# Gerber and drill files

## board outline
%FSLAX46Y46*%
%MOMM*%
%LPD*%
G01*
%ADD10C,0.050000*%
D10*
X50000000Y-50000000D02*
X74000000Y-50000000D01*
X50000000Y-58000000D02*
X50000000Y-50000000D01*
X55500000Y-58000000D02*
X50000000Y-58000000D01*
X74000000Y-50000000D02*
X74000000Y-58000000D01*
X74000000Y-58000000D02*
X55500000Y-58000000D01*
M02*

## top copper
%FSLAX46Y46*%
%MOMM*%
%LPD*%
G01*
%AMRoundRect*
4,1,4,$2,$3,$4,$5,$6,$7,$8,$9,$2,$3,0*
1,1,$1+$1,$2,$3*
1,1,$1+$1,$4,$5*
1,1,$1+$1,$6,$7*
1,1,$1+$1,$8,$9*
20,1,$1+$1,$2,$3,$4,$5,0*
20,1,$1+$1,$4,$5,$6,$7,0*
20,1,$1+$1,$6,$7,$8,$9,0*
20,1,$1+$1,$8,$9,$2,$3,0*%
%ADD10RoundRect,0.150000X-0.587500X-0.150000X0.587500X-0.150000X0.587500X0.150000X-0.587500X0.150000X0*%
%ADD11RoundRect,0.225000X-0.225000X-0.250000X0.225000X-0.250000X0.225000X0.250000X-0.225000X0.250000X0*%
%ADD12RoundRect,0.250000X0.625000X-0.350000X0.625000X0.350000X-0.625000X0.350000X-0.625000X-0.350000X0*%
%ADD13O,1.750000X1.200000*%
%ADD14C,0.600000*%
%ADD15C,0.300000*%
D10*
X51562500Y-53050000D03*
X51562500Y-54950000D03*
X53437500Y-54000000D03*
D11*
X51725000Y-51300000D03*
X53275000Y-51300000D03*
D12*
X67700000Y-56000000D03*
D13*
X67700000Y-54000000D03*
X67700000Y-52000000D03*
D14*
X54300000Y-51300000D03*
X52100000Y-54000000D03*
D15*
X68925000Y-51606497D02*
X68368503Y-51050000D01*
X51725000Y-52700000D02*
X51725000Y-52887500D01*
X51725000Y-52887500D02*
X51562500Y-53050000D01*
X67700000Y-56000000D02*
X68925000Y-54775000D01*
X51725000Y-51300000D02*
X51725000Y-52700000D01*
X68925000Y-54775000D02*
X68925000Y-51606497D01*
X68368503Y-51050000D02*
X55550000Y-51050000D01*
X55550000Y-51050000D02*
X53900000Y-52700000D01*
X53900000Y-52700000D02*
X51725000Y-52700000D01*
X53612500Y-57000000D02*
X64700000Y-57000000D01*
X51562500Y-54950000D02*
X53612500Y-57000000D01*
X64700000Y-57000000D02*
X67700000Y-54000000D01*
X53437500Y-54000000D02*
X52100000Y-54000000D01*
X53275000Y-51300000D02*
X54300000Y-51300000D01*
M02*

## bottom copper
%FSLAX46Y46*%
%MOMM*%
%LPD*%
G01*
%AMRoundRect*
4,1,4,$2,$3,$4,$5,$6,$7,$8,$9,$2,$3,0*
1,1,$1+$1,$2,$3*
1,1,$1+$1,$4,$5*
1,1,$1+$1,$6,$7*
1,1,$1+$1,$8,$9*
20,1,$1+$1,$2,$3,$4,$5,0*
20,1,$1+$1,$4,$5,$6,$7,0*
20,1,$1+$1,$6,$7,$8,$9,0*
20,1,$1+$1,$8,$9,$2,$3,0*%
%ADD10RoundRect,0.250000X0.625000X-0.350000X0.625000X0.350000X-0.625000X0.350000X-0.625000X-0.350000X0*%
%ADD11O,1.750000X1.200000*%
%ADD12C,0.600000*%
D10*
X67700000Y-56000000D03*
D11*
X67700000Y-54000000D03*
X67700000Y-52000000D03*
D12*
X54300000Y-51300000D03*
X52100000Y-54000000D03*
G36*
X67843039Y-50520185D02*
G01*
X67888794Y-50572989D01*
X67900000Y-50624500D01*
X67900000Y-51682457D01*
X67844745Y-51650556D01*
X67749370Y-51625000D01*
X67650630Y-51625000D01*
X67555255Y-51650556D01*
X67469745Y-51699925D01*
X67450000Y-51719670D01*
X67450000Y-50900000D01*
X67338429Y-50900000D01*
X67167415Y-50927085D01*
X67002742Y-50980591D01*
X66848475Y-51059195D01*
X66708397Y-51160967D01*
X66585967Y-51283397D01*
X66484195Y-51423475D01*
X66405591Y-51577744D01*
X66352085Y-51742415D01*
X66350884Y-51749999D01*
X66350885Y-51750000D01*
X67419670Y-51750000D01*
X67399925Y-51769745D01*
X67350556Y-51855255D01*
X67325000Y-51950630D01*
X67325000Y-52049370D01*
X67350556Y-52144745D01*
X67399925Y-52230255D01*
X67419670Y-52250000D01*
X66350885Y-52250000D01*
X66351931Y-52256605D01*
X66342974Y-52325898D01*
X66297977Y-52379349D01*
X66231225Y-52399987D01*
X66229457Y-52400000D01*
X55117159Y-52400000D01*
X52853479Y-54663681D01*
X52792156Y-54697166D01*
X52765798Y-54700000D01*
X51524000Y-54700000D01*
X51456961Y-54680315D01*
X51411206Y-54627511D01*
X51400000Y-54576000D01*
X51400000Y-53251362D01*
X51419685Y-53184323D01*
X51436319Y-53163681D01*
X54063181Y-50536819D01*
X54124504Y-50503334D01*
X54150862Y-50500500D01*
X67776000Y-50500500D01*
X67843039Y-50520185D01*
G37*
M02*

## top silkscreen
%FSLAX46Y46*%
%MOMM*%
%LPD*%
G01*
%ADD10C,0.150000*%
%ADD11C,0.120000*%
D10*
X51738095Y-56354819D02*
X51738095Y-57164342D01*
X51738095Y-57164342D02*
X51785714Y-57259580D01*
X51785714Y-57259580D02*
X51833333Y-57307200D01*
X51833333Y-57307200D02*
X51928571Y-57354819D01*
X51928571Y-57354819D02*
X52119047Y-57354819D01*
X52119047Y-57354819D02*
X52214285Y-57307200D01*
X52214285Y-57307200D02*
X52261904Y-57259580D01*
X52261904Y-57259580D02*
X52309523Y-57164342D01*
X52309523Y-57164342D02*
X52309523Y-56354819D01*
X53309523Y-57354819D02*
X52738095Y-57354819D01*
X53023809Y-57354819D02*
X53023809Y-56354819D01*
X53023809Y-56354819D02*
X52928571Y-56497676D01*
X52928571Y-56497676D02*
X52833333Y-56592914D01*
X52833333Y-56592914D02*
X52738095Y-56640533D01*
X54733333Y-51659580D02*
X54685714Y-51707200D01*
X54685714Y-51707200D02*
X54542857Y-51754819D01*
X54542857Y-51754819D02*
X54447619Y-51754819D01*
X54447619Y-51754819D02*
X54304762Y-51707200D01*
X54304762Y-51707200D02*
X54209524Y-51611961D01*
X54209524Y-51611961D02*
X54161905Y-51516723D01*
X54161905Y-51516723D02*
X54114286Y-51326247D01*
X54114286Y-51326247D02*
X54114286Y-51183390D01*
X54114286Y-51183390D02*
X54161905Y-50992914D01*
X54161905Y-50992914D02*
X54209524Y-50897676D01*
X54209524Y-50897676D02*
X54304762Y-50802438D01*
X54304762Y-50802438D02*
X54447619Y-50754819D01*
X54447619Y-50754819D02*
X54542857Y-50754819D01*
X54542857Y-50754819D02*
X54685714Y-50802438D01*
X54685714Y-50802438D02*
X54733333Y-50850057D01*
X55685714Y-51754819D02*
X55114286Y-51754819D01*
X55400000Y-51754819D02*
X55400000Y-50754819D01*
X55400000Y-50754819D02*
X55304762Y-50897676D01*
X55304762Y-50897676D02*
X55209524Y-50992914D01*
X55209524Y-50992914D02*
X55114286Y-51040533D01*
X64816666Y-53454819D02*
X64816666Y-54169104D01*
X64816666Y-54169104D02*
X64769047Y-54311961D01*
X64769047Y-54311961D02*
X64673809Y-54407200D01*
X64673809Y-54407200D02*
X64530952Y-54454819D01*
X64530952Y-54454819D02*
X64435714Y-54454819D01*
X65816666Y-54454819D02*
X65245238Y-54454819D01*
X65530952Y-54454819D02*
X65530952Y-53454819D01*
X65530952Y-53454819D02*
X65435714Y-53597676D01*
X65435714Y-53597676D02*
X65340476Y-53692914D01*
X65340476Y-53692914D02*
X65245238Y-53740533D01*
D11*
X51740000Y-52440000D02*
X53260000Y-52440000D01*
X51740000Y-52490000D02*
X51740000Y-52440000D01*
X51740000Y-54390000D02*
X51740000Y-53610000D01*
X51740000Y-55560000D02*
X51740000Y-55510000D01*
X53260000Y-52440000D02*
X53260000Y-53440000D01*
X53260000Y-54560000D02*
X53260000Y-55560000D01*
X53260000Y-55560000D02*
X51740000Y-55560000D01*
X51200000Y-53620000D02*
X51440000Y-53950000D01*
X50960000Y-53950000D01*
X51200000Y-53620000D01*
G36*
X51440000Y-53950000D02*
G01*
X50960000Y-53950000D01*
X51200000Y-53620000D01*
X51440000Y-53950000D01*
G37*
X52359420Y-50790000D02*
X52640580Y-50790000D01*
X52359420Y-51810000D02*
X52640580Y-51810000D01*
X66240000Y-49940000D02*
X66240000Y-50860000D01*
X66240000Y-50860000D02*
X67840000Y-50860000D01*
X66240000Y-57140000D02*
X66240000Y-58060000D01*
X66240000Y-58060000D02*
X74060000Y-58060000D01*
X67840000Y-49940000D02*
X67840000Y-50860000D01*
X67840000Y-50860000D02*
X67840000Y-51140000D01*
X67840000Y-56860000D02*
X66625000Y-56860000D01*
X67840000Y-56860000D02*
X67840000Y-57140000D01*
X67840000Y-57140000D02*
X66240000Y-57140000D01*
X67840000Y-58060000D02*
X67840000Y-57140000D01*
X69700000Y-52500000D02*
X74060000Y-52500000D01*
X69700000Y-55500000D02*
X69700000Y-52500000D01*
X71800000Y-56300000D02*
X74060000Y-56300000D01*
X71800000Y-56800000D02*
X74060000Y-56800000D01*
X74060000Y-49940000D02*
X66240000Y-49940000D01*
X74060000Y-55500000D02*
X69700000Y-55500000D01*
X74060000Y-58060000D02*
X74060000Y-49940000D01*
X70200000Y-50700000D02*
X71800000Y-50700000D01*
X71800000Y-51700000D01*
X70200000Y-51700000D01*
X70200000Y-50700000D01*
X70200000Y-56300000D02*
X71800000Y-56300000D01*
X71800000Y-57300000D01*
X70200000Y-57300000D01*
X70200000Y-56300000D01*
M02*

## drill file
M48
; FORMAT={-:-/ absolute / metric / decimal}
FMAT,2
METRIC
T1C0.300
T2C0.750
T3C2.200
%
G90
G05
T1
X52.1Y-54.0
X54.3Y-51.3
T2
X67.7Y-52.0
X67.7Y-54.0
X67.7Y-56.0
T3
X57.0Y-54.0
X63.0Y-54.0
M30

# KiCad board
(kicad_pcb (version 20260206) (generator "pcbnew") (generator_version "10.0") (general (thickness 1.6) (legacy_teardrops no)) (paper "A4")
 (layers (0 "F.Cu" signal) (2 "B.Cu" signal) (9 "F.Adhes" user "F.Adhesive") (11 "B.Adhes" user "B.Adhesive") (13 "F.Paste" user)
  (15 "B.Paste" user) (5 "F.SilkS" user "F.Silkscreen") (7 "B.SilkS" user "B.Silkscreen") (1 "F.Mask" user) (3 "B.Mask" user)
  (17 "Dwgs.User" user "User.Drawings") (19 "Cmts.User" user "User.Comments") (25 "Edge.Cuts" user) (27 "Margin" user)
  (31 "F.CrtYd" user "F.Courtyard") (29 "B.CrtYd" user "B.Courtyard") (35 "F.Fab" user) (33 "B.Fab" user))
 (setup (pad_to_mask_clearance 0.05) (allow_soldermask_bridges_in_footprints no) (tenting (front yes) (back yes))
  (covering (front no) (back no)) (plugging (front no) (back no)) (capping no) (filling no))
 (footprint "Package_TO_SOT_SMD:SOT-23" (layer "F.Cu") (at 52.5 54)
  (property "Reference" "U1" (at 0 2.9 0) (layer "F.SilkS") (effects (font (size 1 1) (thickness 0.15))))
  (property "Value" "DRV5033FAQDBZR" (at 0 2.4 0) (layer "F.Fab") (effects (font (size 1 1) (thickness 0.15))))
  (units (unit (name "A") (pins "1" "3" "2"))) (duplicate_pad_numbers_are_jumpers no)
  (fp_line (start -0.76 -1.56) (end 0.76 -1.56) (stroke (width 0.12) (type solid)) (layer "F.SilkS"))
  (fp_line (start -0.76 -1.51) (end -0.76 -1.56) (stroke (width 0.12) (type solid)) (layer "F.SilkS"))
  (fp_line (start -0.76 0.39) (end -0.76 -0.39) (stroke (width 0.12) (type solid)) (layer "F.SilkS"))
  (fp_line (start -0.76 1.56) (end -0.76 1.51) (stroke (width 0.12) (type solid)) (layer "F.SilkS"))
  (fp_line (start 0.76 -1.56) (end 0.76 -0.56) (stroke (width 0.12) (type solid)) (layer "F.SilkS"))
  (fp_line (start 0.76 0.56) (end 0.76 1.56) (stroke (width 0.12) (type solid)) (layer "F.SilkS"))
  (fp_line (start 0.76 1.56) (end -0.76 1.56) (stroke (width 0.12) (type solid)) (layer "F.SilkS"))
  (fp_poly (pts (xy -1.3 -0.38) (xy -1.06 -0.05) (xy -1.54 -0.05)) (stroke (width 0.12) (type solid)) (fill yes) (layer "F.SilkS"))
  (pad "1" smd roundrect (at -0.9375 -0.95) (size 1.475 0.6) (layers "F.Cu" "F.Mask" "F.Paste") (roundrect_rratio 0.25) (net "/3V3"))
  (pad "2" smd roundrect (at -0.9375 0.95) (size 1.475 0.6) (layers "F.Cu" "F.Mask" "F.Paste") (roundrect_rratio 0.25) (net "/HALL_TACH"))
  (pad "3" smd roundrect (at 0.9375 0) (size 1.475 0.6) (layers "F.Cu" "F.Mask" "F.Paste") (roundrect_rratio 0.25) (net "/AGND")))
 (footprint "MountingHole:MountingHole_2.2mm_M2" (layer "F.Cu") (at 63 54)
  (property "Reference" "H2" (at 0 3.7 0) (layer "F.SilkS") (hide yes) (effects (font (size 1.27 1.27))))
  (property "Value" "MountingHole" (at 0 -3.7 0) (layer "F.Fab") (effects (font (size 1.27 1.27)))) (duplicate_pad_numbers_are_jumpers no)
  (pad "" np_thru_hole circle (at 0 0) (size 2.2 2.2) (drill 2.2) (layers "*.Cu" "*.Mask")))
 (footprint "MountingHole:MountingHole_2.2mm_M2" (layer "F.Cu") (at 57 54)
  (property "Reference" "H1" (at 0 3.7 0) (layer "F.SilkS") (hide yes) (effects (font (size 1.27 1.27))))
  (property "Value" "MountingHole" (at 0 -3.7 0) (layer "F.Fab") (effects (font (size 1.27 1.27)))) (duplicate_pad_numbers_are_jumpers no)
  (pad "" np_thru_hole circle (at 0 0) (size 2.2 2.2) (drill 2.2) (layers "*.Cu" "*.Mask")))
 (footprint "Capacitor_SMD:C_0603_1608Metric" (layer "F.Cu") (at 52.5 51.3)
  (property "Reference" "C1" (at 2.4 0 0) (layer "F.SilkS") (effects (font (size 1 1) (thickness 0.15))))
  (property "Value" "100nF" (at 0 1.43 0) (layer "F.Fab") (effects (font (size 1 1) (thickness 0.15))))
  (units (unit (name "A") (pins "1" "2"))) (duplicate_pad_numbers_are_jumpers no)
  (fp_line (start -0.14058 -0.51) (end 0.14058 -0.51) (stroke (width 0.12) (type solid)) (layer "F.SilkS"))
  (fp_line (start -0.14058 0.51) (end 0.14058 0.51) (stroke (width 0.12) (type solid)) (layer "F.SilkS"))
  (pad "1" smd roundrect (at -0.775 0) (size 0.9 0.95) (layers "F.Cu" "F.Mask" "F.Paste") (roundrect_rratio 0.25) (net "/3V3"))
  (pad "2" smd roundrect (at 0.775 0) (size 0.9 0.95) (layers "F.Cu" "F.Mask" "F.Paste") (roundrect_rratio 0.25) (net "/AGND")))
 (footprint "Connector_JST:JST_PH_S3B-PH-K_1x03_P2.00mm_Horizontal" (layer "F.Cu") (at 67.7 56 90)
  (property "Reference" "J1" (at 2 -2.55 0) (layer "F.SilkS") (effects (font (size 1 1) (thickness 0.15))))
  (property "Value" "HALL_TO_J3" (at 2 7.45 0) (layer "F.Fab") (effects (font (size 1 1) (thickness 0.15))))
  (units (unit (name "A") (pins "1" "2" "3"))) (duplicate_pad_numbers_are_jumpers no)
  (fp_line (start 6.06 -1.46) (end 5.14 -1.46) (stroke (width 0.12) (type solid)) (layer "F.SilkS"))
  (fp_line (start 5.14 -1.46) (end 5.14 0.14) (stroke (width 0.12) (type solid)) (layer "F.SilkS"))
  (fp_line (start -1.14 -1.46) (end -2.06 -1.46) (stroke (width 0.12) (type solid)) (layer "F.SilkS"))
  (fp_line (start -2.06 -1.46) (end -2.06 6.36) (stroke (width 0.12) (type solid)) (layer "F.SilkS"))
  (fp_line (start 6.06 0.14) (end 5.14 0.14) (stroke (width 0.12) (type solid)) (layer "F.SilkS"))
  (fp_line (start 5.14 0.14) (end 4.86 0.14) (stroke (width 0.12) (type solid)) (layer "F.SilkS"))
  (fp_line (start -0.86 0.14) (end -0.86 -1.075) (stroke (width 0.12) (type solid)) (layer "F.SilkS"))
  (fp_line (start -0.86 0.14) (end -1.14 0.14) (stroke (width 0.12) (type solid)) (layer "F.SilkS"))
  (fp_line (start -1.14 0.14) (end -1.14 -1.46) (stroke (width 0.12) (type solid)) (layer "F.SilkS"))
  (fp_line (start -2.06 0.14) (end -1.14 0.14) (stroke (width 0.12) (type solid)) (layer "F.SilkS"))
  (fp_line (start 3.5 2) (end 3.5 6.36) (stroke (width 0.12) (type solid)) (layer "F.SilkS"))
  (fp_line (start 0.5 2) (end 3.5 2) (stroke (width 0.12) (type solid)) (layer "F.SilkS"))
  (fp_line (start -0.3 4.1) (end -0.3 6.36) (stroke (width 0.12) (type solid)) (layer "F.SilkS"))
  (fp_line (start -0.8 4.1) (end -0.8 6.36) (stroke (width 0.12) (type solid)) (layer "F.SilkS"))
  (fp_line (start 6.06 6.36) (end 6.06 -1.46) (stroke (width 0.12) (type solid)) (layer "F.SilkS"))
  (fp_line (start 0.5 6.36) (end 0.5 2) (stroke (width 0.12) (type solid)) (layer "F.SilkS"))
  (fp_line (start -2.06 6.36) (end 6.06 6.36) (stroke (width 0.12) (type solid)) (layer "F.SilkS"))
  (fp_rect (start 4.3 2.5) (end 5.3 4.1) (stroke (width 0.12) (type solid)) (fill no) (layer "F.SilkS"))
  (fp_rect (start -1.3 2.5) (end -0.3 4.1) (stroke (width 0.12) (type solid)) (fill no) (layer "F.SilkS"))
  (pad "1" thru_hole roundrect (at 0 0 90) (size 1.2 1.75) (drill 0.75) (layers "*.Cu" "*.Mask") (remove_unused_layers no)
   (roundrect_rratio 0.208333) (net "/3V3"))
  (pad "2" thru_hole oval (at 2 0 90) (size 1.2 1.75) (drill 0.75) (layers "*.Cu" "*.Mask") (remove_unused_layers no) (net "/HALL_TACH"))
  (pad "3" thru_hole oval (at 4 0 90) (size 1.2 1.75) (drill 0.75) (layers "*.Cu" "*.Mask") (remove_unused_layers no) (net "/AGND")))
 (gr_line (start 50 50) (end 74 50) (stroke (width 0.05) (type solid)) (layer "Edge.Cuts"))
 (gr_line (start 50 58) (end 50 50) (stroke (width 0.05) (type solid)) (layer "Edge.Cuts"))
 (gr_line (start 55.5 58) (end 50 58) (stroke (width 0.05) (type solid)) (layer "Edge.Cuts"))
 (gr_line (start 74 50) (end 74 58) (stroke (width 0.05) (type solid)) (layer "Edge.Cuts"))
 (gr_line (start 74 58) (end 55.5 58) (stroke (width 0.05) (type solid)) (layer "Edge.Cuts"))
 (segment (start 68.925 51.606497) (end 68.368503 51.05) (width 0.3) (layer "F.Cu") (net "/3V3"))
 (segment (start 51.725 52.7) (end 51.725 52.8875) (width 0.3) (layer "F.Cu") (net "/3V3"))
 (segment (start 51.725 52.8875) (end 51.5625 53.05) (width 0.3) (layer "F.Cu") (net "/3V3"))
 (segment (start 67.7 56) (end 68.925 54.775) (width 0.3) (layer "F.Cu") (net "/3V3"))
 (segment (start 51.725 51.3) (end 51.725 52.7) (width 0.3) (layer "F.Cu") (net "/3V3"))
 (segment (start 68.925 54.775) (end 68.925 51.606497) (width 0.3) (layer "F.Cu") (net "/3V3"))
 (segment (start 68.368503 51.05) (end 55.55 51.05) (width 0.3) (layer "F.Cu") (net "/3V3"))
 (segment (start 55.55 51.05) (end 53.9 52.7) (width 0.3) (layer "F.Cu") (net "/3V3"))
 (segment (start 53.9 52.7) (end 51.725 52.7) (width 0.3) (layer "F.Cu") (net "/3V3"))
 (segment (start 53.6125 57) (end 64.7 57) (width 0.3) (layer "F.Cu") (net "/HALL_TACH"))
 (segment (start 51.5625 54.95) (end 53.6125 57) (width 0.3) (layer "F.Cu") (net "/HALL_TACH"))
 (segment (start 64.7 57) (end 67.7 54) (width 0.3) (layer "F.Cu") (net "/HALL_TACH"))
 (segment (start 53.4375 54) (end 52.1 54) (width 0.3) (layer "F.Cu") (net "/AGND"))
 (segment (start 53.275 51.3) (end 54.3 51.3) (width 0.3) (layer "F.Cu") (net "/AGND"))
 (via (at 54.3 51.3) (size 0.6) (drill 0.3) (layers "F.Cu" "B.Cu") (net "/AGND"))
 (via (at 52.1 54) (size 0.6) (drill 0.3) (layers "F.Cu" "B.Cu") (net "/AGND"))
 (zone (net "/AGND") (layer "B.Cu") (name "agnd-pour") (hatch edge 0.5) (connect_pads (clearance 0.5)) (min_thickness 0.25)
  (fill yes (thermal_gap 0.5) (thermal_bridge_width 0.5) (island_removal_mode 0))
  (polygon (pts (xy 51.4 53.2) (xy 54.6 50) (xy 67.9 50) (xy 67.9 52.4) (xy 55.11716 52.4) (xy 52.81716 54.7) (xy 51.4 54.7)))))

